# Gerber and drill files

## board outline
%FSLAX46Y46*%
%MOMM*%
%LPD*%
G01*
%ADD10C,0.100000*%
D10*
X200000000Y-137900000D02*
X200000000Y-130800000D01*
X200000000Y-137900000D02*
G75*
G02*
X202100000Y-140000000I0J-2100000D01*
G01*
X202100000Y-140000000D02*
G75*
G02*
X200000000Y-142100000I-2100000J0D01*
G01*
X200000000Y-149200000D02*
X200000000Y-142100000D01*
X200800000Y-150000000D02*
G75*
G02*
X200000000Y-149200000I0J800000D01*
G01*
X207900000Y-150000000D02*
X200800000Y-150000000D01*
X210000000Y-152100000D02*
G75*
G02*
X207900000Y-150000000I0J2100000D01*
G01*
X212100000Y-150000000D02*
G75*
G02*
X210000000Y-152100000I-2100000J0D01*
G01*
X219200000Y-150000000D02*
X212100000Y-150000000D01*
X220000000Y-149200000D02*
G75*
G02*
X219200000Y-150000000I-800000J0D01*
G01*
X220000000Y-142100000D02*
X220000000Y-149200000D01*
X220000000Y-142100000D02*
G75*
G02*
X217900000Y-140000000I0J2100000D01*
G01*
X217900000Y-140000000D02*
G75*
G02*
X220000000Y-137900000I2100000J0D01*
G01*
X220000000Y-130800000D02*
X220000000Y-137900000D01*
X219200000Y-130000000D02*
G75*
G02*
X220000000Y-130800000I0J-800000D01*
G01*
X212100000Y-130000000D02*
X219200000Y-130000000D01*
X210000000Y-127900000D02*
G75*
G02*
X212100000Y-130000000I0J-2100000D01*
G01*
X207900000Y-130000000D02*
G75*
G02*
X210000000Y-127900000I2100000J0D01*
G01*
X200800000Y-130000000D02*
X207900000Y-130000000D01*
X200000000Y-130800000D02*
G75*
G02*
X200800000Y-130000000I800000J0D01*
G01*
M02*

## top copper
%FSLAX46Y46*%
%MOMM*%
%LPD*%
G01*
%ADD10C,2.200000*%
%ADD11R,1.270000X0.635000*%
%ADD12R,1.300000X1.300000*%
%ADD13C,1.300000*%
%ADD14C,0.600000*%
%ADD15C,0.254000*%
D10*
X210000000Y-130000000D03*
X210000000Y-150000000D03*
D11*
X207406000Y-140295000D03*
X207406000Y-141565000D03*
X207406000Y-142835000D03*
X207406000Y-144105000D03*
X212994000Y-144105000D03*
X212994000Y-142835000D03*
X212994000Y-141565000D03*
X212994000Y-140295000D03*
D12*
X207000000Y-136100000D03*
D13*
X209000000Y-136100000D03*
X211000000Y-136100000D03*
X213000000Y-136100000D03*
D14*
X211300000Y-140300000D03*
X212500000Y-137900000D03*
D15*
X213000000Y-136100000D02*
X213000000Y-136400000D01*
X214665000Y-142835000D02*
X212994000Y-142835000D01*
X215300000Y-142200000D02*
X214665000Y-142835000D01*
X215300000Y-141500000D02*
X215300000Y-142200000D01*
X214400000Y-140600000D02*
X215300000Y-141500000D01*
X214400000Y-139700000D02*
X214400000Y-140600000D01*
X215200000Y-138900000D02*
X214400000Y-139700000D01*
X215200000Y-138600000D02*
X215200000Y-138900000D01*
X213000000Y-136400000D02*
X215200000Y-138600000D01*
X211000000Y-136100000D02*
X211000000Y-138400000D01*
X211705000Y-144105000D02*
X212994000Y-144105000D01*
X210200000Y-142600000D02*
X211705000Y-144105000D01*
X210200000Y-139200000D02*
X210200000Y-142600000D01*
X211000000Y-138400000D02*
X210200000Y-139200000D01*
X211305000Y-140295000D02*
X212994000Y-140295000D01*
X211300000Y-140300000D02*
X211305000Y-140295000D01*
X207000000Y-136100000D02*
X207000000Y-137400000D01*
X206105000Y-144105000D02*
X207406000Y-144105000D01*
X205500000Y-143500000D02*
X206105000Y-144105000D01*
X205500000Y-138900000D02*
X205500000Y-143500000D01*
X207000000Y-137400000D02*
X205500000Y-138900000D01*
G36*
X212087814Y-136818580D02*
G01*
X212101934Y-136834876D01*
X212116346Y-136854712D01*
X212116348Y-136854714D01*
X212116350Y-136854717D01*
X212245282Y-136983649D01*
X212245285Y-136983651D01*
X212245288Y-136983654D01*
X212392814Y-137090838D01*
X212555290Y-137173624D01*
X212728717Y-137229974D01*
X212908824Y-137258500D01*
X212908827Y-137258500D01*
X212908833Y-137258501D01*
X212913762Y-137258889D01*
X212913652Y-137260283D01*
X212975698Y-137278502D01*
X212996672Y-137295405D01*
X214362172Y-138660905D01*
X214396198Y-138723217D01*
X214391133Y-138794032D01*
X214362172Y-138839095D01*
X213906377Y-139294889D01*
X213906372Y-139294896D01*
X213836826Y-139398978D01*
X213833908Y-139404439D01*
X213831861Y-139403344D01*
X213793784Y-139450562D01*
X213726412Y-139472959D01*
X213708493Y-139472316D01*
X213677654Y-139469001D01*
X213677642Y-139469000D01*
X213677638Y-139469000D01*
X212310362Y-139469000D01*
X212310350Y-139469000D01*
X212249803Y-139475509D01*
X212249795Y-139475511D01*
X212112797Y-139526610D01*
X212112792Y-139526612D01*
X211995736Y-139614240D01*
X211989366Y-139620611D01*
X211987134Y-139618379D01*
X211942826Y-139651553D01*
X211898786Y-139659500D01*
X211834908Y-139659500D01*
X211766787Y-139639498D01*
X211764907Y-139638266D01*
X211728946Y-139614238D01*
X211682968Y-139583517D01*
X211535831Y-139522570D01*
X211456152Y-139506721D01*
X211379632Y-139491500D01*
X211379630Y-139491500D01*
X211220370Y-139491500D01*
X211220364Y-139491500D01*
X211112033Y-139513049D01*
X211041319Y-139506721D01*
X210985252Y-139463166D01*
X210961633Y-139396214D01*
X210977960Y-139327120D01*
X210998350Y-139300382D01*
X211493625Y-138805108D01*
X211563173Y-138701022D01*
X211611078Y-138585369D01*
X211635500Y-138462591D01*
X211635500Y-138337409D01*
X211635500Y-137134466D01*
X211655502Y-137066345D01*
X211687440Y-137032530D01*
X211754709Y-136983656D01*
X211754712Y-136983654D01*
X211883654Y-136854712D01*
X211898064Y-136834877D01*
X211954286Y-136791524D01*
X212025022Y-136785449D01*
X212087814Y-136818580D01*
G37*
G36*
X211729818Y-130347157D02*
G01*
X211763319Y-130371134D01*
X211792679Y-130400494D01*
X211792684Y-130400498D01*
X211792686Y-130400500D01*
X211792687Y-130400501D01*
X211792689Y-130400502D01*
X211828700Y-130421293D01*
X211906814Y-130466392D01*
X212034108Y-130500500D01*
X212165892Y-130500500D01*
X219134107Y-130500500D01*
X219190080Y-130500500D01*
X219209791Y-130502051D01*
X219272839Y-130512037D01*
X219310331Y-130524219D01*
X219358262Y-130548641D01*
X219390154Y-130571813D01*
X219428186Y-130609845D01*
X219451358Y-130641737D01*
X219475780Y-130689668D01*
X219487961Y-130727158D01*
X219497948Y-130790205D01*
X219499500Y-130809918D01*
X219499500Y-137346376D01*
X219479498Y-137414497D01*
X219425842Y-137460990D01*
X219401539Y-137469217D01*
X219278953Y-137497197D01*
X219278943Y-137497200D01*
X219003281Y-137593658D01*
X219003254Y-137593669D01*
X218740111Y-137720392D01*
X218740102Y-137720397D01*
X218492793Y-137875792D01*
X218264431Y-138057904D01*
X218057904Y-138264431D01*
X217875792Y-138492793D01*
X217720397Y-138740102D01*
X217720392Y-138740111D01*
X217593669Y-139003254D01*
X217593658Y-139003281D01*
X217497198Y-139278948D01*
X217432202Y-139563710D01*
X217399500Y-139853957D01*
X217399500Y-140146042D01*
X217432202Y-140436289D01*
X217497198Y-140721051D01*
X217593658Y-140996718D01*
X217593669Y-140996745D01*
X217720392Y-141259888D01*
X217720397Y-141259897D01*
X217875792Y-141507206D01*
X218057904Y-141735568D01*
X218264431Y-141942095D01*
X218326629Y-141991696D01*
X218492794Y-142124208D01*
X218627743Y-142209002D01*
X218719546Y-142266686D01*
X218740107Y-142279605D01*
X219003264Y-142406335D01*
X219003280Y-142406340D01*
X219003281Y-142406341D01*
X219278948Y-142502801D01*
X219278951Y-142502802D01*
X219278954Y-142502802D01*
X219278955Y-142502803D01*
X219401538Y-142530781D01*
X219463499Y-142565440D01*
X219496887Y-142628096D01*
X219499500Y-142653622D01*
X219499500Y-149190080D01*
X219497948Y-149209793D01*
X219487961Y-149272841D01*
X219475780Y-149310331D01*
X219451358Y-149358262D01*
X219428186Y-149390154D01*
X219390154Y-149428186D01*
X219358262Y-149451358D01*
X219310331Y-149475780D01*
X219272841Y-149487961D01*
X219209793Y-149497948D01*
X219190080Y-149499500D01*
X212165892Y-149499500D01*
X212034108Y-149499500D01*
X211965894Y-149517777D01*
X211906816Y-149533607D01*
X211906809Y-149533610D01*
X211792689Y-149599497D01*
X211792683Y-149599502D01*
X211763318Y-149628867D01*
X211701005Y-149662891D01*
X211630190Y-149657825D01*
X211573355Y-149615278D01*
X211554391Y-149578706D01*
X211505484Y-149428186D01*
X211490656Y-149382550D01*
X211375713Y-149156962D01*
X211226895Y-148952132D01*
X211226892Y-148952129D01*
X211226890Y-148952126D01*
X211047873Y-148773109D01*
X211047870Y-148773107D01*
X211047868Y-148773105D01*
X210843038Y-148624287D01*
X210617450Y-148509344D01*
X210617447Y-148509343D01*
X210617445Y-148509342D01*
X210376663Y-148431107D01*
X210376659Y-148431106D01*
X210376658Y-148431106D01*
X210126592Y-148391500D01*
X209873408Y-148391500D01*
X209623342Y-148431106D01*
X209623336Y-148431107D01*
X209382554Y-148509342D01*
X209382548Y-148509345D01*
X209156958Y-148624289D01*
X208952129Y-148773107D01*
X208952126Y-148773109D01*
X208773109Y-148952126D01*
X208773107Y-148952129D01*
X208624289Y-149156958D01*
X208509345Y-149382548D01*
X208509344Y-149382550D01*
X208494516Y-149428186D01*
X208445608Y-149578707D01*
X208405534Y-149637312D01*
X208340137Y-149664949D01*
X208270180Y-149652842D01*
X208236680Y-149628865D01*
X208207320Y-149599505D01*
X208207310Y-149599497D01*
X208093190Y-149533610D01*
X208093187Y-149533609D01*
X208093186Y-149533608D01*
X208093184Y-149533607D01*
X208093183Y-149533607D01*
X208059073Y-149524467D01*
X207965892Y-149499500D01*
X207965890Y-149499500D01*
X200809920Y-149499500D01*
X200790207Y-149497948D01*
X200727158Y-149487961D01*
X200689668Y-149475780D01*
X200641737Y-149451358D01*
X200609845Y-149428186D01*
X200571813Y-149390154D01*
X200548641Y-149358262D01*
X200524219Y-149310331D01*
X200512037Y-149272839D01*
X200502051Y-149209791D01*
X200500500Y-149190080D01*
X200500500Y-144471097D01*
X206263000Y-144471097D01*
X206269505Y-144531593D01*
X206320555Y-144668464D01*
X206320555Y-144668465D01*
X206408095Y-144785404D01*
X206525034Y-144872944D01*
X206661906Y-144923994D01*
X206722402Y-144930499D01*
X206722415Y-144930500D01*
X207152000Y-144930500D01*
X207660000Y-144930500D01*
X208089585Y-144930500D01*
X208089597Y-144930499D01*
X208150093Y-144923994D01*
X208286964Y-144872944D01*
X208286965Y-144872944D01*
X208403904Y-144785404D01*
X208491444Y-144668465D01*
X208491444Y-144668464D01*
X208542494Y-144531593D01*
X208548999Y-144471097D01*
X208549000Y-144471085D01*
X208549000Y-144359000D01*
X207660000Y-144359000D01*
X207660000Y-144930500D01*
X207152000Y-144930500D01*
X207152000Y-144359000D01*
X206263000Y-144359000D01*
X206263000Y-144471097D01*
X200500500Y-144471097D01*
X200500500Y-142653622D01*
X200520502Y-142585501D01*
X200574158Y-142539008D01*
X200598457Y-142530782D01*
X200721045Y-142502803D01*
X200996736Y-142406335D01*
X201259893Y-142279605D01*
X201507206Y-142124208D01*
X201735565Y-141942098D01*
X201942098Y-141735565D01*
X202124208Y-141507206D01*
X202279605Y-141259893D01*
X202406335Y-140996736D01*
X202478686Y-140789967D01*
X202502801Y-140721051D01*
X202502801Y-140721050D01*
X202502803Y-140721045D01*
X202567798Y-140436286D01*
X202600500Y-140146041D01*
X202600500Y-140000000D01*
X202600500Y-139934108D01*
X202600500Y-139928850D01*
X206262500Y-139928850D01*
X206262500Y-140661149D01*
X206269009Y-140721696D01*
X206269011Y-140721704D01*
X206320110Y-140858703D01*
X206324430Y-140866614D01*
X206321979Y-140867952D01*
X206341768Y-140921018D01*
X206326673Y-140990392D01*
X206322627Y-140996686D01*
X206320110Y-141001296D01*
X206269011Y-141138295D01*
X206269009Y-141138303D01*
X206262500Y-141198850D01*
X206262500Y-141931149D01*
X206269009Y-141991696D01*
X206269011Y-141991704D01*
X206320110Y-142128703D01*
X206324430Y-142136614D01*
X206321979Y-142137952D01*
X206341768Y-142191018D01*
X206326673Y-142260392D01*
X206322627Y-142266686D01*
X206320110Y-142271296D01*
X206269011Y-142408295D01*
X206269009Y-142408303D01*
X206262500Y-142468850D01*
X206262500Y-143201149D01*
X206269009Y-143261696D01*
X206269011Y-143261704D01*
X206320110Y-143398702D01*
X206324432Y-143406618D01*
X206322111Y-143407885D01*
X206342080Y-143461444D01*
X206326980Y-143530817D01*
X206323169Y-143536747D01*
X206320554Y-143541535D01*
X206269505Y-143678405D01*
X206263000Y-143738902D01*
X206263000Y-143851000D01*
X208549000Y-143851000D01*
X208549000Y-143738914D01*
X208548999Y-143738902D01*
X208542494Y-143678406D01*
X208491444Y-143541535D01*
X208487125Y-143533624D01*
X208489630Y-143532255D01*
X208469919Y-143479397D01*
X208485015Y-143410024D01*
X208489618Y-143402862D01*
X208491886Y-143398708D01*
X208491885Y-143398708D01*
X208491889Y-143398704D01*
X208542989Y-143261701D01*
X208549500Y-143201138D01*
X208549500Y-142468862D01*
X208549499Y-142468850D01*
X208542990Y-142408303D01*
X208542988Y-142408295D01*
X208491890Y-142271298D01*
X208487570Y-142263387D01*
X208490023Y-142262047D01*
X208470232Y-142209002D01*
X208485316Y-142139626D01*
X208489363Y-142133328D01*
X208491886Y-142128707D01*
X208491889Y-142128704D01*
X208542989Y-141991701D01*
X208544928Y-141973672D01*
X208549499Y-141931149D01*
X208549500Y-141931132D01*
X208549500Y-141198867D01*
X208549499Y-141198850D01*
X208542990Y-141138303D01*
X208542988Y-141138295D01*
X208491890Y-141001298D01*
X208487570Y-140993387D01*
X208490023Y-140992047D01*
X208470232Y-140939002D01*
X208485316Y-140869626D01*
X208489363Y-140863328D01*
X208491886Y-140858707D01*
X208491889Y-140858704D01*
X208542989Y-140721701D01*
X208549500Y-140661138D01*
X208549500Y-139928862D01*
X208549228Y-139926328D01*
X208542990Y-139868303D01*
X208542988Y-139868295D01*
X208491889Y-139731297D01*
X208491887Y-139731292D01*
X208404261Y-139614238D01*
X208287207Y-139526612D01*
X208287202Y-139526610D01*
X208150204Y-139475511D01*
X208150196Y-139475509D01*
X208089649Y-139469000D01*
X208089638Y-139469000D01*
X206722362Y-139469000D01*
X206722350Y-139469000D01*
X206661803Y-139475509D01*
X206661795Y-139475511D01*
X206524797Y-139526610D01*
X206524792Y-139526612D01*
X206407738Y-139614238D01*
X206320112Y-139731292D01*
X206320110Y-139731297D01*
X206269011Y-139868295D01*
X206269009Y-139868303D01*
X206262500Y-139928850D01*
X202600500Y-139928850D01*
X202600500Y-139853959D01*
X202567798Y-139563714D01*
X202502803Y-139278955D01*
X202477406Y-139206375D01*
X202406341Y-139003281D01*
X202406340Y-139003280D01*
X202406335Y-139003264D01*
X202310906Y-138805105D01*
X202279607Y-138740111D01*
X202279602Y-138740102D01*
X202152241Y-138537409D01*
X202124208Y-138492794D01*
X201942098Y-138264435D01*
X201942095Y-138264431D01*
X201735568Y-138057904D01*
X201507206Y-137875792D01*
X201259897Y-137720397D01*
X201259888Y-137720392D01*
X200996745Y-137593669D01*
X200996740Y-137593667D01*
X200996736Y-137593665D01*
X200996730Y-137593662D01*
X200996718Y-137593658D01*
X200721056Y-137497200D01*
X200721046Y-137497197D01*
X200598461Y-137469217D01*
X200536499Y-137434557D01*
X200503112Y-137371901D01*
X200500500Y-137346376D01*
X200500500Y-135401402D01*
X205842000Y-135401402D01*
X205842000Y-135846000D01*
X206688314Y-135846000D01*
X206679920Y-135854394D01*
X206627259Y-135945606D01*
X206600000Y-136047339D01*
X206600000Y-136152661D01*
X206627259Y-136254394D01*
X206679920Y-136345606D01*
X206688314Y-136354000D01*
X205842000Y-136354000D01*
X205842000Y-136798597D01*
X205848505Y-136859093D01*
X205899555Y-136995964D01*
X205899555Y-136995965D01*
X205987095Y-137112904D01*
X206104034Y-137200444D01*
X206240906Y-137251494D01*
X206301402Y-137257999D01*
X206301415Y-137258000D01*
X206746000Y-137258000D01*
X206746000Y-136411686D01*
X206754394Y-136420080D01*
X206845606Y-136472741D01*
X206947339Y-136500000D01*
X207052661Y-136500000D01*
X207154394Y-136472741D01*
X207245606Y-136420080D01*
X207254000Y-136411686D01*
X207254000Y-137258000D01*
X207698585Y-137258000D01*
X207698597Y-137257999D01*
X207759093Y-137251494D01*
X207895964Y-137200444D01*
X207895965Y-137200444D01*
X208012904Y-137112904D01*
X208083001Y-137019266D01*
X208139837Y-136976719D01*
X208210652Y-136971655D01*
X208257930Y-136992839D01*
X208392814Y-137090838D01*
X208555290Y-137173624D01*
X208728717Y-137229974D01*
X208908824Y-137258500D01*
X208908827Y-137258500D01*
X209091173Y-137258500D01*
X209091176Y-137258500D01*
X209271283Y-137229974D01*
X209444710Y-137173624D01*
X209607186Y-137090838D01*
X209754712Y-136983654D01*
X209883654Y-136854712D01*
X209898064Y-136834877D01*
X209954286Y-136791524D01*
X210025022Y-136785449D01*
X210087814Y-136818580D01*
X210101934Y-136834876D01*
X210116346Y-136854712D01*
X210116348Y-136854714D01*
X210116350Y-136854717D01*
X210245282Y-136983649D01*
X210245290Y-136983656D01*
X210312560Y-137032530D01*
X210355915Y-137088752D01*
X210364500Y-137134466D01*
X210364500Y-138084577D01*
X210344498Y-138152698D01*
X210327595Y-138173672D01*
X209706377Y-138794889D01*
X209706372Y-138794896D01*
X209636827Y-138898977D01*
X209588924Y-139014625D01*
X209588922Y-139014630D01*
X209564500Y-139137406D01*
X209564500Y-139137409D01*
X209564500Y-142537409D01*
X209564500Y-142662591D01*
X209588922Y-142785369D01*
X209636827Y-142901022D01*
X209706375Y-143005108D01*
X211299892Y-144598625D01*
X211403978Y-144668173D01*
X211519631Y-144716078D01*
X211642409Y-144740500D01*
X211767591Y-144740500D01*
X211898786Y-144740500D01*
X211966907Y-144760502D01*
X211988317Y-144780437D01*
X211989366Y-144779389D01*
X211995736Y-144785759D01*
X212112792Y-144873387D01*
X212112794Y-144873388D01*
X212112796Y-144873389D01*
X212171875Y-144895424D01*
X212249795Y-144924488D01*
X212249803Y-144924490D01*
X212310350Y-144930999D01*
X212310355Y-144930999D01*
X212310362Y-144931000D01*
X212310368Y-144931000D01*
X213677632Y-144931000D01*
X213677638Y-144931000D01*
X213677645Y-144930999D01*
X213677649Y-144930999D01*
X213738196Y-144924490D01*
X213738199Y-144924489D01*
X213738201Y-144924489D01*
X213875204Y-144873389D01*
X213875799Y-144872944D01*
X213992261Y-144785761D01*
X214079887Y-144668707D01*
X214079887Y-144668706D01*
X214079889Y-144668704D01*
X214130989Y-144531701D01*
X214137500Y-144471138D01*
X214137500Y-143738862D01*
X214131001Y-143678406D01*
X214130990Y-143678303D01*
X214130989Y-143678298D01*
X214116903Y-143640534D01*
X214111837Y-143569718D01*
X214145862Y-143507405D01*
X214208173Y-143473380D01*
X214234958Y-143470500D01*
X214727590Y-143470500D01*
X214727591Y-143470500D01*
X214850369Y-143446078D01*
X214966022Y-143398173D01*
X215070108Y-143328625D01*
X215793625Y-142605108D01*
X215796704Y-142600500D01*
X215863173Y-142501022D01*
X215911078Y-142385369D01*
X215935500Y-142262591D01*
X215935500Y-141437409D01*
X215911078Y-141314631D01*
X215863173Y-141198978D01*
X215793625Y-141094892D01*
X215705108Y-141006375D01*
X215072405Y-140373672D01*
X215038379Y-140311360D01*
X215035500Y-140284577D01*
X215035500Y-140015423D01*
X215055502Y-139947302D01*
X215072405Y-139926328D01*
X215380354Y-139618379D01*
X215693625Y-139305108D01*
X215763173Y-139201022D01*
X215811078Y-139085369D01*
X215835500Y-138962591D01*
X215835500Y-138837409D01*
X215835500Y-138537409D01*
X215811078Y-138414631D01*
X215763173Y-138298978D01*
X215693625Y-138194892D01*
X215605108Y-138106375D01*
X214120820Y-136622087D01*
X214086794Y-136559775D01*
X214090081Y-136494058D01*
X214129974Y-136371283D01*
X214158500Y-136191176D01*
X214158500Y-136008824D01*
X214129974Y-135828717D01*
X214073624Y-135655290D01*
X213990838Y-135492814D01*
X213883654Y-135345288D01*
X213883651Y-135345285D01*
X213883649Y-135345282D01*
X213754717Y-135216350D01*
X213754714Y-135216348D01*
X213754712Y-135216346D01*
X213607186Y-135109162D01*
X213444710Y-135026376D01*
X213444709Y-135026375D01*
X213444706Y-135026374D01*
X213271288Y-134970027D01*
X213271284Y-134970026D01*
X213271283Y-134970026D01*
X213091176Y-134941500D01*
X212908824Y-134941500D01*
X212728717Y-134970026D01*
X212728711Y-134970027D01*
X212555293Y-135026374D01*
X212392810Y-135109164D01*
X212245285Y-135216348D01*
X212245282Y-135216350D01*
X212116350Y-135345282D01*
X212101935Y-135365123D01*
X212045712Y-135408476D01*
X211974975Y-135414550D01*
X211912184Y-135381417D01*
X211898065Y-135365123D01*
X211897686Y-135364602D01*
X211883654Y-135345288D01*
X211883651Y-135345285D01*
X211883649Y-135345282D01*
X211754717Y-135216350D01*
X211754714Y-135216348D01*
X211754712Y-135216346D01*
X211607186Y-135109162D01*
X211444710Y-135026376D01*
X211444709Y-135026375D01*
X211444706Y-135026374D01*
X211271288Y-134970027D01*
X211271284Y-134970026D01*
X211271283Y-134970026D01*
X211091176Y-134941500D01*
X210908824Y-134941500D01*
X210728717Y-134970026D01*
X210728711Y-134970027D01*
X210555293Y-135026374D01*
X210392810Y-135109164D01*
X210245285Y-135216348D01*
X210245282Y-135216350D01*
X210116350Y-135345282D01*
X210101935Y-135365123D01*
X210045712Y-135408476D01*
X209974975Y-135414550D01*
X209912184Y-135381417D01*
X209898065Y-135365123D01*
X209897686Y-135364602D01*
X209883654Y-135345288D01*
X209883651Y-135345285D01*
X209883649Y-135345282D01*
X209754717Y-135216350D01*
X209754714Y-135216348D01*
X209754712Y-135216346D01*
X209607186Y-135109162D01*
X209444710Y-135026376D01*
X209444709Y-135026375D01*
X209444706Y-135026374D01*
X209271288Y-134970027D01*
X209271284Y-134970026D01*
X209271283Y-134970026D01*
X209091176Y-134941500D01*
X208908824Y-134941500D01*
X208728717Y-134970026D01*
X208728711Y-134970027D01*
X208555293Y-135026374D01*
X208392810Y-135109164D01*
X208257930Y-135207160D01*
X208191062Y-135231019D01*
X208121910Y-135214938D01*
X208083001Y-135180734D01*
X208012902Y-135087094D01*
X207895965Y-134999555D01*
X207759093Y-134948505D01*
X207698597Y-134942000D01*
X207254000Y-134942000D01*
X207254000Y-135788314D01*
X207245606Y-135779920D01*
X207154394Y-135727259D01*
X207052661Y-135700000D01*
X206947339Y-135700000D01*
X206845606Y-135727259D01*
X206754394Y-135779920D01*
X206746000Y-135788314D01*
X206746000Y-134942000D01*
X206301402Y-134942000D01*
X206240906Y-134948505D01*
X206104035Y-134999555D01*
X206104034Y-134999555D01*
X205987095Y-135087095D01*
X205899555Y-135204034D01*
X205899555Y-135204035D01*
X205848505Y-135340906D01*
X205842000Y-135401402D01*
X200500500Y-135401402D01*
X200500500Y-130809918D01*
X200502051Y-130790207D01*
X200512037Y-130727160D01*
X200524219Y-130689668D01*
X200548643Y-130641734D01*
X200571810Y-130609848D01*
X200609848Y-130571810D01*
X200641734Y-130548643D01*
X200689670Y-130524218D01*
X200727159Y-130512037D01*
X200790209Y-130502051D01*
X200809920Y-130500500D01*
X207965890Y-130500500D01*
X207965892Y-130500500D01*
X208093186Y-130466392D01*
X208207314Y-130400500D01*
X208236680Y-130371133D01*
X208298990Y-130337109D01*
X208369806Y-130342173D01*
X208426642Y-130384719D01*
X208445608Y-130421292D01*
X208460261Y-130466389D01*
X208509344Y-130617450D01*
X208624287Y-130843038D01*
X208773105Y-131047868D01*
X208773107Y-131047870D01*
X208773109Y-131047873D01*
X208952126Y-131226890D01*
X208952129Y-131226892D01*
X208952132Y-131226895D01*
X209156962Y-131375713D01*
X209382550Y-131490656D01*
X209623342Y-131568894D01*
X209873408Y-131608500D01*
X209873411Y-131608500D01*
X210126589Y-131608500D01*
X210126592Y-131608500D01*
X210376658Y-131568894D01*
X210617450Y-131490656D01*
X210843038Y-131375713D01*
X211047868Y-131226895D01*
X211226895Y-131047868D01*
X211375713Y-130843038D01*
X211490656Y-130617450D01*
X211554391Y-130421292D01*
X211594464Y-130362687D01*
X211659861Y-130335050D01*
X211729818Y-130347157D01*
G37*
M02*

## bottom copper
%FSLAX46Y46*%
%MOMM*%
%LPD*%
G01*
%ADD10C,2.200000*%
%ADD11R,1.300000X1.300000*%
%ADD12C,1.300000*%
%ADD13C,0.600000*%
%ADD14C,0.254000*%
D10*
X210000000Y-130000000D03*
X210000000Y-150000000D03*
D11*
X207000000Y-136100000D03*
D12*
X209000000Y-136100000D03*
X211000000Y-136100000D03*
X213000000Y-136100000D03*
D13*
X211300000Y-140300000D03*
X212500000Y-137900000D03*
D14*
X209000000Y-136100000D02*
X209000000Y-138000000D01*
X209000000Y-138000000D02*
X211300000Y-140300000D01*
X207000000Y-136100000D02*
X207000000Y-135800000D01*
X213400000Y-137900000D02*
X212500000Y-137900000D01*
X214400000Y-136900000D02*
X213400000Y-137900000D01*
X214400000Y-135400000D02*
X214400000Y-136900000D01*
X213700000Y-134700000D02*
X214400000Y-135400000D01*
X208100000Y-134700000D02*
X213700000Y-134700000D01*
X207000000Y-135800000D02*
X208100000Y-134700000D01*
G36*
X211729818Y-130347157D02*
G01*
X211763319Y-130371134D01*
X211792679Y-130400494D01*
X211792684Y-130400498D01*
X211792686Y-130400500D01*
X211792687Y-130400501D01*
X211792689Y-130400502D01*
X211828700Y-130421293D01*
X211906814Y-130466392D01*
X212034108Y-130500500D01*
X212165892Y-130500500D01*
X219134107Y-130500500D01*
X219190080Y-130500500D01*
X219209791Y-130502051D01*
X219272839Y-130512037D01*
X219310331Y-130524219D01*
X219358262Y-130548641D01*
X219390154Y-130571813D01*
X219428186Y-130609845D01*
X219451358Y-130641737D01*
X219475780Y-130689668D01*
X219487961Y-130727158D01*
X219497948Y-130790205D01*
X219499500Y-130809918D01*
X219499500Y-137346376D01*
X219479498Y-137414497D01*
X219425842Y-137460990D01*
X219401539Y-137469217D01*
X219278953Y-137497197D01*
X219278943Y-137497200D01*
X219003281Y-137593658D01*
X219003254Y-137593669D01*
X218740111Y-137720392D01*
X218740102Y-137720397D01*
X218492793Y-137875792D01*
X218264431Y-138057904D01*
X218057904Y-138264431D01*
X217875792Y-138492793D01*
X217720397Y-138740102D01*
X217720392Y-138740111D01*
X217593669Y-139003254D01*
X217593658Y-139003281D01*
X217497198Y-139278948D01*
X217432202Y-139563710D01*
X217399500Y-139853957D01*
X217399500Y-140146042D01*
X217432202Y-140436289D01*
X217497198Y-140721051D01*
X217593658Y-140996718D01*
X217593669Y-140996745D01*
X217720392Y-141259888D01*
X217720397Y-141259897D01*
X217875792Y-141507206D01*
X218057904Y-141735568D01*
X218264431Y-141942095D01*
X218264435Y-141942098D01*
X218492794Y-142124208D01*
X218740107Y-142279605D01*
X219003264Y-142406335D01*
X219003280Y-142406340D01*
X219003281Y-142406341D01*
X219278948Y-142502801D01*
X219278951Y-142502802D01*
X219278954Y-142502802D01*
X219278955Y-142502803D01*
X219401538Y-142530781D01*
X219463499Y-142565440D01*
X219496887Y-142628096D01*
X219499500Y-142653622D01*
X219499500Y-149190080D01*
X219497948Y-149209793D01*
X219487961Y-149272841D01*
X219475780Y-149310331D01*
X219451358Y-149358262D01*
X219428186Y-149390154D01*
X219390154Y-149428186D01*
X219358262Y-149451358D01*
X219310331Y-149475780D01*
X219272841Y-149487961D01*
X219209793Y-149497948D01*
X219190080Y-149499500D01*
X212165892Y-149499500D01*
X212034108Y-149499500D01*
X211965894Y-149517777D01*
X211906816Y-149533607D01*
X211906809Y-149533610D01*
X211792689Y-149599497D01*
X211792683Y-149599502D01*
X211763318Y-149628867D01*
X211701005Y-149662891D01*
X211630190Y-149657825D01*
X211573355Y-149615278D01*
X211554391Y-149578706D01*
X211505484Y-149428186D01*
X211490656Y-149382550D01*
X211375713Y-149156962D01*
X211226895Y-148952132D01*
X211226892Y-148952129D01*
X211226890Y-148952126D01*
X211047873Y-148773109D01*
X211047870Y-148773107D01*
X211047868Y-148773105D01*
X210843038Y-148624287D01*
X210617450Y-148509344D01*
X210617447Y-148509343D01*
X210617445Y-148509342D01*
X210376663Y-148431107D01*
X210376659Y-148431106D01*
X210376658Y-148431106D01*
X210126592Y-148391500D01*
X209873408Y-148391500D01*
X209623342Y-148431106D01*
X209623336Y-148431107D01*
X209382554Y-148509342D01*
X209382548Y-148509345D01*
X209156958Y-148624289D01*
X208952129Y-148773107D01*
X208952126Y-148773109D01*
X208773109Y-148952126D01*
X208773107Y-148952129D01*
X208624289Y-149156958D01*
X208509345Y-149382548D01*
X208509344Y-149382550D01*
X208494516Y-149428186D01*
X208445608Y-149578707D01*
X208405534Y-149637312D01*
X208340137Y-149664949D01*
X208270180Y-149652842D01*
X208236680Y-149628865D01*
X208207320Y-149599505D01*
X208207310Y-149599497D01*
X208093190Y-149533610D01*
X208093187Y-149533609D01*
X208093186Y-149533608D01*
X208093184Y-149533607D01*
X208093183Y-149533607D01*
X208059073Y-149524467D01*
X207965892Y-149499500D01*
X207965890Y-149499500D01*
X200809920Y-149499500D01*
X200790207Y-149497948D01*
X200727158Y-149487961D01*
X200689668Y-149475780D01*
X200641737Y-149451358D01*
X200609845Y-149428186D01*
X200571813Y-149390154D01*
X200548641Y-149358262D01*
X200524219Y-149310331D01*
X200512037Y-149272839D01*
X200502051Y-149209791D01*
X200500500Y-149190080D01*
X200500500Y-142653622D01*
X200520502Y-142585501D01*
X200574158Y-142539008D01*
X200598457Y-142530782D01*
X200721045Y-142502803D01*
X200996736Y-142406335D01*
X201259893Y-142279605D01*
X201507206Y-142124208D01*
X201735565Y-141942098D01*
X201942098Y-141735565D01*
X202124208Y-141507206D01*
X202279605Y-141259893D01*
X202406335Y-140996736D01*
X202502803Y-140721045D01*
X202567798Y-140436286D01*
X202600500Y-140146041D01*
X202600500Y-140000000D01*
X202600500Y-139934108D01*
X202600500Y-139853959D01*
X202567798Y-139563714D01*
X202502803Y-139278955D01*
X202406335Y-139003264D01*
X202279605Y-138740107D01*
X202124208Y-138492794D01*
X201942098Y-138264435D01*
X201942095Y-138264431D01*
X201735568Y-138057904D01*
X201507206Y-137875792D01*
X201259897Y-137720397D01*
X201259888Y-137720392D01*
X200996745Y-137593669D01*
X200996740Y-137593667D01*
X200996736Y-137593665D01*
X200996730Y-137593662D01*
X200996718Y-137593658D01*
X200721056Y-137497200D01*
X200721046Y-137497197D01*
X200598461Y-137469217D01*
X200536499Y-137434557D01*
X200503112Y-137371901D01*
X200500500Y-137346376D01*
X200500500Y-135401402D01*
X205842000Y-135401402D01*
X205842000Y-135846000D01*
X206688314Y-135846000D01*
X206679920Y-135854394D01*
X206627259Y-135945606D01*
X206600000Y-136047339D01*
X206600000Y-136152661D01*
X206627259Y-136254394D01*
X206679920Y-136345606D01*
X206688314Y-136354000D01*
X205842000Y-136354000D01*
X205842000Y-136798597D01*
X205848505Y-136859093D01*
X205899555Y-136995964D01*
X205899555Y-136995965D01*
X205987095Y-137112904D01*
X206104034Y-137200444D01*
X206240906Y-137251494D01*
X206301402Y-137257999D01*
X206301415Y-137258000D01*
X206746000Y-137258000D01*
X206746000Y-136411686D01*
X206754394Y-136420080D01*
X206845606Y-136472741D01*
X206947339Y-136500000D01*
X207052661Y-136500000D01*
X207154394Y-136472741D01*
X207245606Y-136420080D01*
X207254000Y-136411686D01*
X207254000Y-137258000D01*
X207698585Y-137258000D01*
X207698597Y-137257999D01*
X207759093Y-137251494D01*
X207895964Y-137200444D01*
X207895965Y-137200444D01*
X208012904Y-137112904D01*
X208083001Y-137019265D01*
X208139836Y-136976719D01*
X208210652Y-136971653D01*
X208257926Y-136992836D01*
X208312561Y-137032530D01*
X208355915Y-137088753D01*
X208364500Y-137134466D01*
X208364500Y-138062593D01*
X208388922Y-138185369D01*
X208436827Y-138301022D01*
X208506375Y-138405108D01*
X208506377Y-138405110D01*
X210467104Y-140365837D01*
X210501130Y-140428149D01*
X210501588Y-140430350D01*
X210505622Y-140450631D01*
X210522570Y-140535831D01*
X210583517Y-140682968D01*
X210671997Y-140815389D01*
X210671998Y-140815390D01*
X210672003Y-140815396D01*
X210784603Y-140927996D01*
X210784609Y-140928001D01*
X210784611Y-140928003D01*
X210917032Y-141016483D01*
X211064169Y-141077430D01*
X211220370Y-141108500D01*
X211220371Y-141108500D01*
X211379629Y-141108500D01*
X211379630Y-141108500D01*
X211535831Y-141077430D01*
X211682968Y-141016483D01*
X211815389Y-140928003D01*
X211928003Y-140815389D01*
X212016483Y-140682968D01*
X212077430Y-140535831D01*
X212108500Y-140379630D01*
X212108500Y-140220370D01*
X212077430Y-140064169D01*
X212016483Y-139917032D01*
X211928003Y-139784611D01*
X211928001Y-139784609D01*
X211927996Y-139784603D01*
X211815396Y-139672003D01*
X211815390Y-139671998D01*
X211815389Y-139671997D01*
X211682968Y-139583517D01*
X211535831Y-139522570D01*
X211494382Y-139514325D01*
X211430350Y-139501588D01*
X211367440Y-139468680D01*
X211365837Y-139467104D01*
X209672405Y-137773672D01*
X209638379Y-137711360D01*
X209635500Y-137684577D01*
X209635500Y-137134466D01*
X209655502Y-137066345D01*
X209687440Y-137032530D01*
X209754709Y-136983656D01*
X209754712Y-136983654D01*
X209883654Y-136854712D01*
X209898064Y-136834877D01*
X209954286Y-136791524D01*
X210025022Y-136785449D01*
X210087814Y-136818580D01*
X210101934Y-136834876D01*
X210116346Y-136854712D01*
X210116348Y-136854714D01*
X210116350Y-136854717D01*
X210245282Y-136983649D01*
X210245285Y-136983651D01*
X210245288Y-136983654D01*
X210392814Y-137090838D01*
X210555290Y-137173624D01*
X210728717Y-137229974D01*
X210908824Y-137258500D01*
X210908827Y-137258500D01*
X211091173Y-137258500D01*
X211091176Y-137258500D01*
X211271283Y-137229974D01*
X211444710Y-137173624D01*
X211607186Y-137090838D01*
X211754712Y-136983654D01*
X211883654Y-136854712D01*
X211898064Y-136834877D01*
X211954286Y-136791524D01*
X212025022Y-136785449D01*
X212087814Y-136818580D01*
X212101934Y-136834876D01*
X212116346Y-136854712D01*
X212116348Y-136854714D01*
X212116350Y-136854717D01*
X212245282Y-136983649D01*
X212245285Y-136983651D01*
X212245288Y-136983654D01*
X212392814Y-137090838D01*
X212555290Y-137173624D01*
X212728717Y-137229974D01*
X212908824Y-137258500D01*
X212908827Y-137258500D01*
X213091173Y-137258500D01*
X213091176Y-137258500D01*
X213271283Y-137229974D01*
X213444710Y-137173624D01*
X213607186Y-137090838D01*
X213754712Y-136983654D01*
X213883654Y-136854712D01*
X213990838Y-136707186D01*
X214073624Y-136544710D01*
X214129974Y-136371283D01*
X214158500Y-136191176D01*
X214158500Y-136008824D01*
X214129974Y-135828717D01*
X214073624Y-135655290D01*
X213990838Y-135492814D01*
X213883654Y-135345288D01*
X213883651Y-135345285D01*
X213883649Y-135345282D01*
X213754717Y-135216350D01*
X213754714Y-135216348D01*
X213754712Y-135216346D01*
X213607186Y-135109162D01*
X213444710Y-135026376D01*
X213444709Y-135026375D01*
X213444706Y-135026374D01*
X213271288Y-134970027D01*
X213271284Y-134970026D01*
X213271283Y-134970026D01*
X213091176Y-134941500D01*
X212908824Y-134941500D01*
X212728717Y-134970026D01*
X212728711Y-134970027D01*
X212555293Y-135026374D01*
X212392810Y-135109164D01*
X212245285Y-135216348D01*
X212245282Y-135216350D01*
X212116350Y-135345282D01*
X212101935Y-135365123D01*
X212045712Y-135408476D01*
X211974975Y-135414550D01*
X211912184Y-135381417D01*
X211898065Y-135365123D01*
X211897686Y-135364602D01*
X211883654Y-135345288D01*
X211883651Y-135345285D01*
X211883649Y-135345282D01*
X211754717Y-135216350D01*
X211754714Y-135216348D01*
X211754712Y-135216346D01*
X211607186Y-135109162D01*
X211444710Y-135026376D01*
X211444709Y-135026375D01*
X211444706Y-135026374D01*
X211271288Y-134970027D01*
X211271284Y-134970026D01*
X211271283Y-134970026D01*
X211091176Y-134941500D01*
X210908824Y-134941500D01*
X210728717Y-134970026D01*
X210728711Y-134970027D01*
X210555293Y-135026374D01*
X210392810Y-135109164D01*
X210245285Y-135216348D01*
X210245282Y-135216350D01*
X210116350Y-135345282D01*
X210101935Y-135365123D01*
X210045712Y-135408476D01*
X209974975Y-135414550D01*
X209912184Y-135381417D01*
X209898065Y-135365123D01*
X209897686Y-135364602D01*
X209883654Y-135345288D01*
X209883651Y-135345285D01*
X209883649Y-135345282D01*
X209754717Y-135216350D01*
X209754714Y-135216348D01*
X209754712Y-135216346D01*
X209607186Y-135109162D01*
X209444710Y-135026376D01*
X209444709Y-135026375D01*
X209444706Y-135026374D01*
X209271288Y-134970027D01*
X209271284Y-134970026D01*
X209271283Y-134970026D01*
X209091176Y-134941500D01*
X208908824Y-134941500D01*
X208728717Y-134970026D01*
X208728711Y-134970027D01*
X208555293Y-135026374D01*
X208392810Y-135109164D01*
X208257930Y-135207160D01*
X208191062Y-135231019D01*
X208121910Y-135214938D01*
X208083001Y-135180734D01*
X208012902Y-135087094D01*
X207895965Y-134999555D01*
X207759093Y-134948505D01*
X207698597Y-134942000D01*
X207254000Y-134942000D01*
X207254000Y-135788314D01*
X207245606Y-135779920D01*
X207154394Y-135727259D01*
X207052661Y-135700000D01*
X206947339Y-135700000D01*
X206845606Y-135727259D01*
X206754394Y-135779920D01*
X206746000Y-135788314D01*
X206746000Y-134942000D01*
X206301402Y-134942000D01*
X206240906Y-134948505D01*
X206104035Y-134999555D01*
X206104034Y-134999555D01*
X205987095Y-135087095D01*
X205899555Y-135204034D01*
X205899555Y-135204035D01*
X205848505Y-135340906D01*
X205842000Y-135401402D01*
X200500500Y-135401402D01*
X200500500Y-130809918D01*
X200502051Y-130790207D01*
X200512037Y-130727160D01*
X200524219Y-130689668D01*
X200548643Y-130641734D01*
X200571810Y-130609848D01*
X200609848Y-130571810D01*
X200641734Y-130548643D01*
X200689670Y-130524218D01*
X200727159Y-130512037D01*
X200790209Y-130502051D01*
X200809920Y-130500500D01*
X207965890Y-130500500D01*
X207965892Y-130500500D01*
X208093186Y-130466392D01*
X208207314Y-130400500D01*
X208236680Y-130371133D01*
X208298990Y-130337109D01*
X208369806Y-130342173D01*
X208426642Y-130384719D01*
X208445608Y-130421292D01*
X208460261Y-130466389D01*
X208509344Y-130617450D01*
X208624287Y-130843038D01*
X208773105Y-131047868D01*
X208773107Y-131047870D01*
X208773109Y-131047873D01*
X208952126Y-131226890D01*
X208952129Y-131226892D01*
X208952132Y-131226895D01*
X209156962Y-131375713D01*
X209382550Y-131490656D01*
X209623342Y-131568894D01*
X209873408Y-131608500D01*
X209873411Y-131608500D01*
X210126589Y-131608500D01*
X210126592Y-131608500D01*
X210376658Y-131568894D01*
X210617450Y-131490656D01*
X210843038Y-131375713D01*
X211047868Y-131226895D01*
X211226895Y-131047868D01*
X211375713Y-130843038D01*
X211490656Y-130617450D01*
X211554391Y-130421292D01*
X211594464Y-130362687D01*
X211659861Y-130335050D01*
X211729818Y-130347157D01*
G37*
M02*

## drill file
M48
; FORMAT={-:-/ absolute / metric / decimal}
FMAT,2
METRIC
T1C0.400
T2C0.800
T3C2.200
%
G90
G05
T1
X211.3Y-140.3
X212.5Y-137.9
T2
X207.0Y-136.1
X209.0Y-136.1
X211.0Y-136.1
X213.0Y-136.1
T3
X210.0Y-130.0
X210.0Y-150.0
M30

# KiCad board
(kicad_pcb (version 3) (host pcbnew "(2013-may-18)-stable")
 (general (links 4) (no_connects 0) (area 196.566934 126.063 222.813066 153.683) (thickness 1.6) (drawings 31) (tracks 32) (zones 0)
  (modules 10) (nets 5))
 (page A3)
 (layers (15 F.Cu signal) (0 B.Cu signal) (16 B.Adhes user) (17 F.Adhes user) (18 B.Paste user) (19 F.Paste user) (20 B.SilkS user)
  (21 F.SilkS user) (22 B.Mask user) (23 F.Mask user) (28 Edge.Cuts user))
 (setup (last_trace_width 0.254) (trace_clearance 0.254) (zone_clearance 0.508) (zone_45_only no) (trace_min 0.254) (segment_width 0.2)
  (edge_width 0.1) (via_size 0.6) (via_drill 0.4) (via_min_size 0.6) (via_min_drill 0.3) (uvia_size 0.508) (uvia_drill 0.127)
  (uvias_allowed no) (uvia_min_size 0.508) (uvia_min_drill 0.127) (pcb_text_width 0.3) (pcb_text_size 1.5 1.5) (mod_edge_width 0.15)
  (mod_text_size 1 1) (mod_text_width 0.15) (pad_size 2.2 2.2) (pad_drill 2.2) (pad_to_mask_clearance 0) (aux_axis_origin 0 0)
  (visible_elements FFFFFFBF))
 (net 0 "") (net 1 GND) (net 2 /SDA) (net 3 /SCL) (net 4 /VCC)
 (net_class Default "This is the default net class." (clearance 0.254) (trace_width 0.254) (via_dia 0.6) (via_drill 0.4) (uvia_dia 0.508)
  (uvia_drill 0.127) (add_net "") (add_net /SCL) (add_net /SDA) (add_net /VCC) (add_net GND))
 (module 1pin (layer F.Cu) (at 210 130)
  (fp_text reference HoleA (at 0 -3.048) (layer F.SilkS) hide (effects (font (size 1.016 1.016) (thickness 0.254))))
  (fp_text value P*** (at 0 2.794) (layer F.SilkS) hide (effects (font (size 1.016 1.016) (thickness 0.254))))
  (pad 1 thru_hole circle (at 0 0) (size 2.2 2.2) (drill 2.2) (layers *.Cu *.Mask F.SilkS)))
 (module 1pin (layer F.Cu) (at 210 150)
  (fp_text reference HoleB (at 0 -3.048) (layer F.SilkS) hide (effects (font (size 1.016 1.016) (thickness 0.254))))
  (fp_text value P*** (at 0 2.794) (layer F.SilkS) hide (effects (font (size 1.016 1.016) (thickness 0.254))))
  (pad 1 thru_hole circle (at 0 0) (size 2.2 2.2) (drill 2.2) (layers *.Cu *.Mask F.SilkS)))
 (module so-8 (layer F.Cu) (at 210.2 142.2 270)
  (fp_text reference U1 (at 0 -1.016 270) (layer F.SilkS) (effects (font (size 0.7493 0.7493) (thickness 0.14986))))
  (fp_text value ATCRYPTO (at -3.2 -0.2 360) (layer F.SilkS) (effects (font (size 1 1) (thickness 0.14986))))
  (pad 1 smd rect (at -1.905 2.794 270) (size 0.635 1.27) (layers F.Cu F.Paste F.Mask))
  (pad 2 smd rect (at -0.635 2.794 270) (size 0.635 1.27) (layers F.Cu F.Paste F.Mask))
  (pad 3 smd rect (at 0.635 2.794 270) (size 0.635 1.27) (layers F.Cu F.Paste F.Mask))
  (pad 4 smd rect (at 1.905 2.794 270) (size 0.635 1.27) (layers F.Cu F.Paste F.Mask) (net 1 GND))
  (pad 5 smd rect (at 1.905 -2.794 270) (size 0.635 1.27) (layers F.Cu F.Paste F.Mask) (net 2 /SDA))
  (pad 6 smd rect (at 0.635 -2.794 270) (size 0.635 1.27) (layers F.Cu F.Paste F.Mask) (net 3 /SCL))
  (pad 7 smd rect (at -0.635 -2.794 270) (size 0.635 1.27) (layers F.Cu F.Paste F.Mask))
  (pad 8 smd rect (at -1.905 -2.794 270) (size 0.635 1.27) (layers F.Cu F.Paste F.Mask) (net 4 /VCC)))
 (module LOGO (layer B.Cu) (at 215.9 146.7)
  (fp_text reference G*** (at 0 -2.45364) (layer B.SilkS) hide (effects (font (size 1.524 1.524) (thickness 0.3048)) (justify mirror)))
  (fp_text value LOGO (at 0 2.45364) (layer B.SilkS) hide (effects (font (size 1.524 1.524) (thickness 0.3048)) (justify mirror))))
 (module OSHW (layer B.Cu) (at 216.3 133.2)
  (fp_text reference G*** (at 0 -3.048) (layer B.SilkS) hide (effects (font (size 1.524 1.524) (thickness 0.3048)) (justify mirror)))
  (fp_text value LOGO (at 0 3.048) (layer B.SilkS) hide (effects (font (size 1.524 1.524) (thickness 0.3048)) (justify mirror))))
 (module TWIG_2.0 (layer F.Cu) (at 210 136.1)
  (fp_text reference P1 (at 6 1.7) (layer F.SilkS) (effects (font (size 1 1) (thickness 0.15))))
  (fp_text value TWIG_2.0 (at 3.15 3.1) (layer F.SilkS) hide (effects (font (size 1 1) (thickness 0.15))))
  (pad 1 thru_hole rect (at -3 0) (size 1.3 1.3) (drill 0.8) (layers *.Cu *.Mask F.SilkS) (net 1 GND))
  (pad 2 thru_hole circle (at -1 0) (size 1.3 1.3) (drill 0.8) (layers *.Cu *.Mask F.SilkS) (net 4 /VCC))
  (pad 3 thru_hole circle (at 1 0) (size 1.3 1.3) (drill 0.8) (layers *.Cu *.Mask F.SilkS) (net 2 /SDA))
  (pad 4 thru_hole circle (at 3 0) (size 1.3 1.3) (drill 0.8) (layers *.Cu *.Mask F.SilkS) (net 3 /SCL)))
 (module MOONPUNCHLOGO (layer B.Cu) (at 211.4 141.4)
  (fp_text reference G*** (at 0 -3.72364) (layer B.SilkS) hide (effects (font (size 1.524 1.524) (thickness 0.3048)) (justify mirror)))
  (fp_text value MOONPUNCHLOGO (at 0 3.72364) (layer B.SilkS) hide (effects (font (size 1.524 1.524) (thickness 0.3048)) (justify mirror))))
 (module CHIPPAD (layer F.Cu) (at 202.9 147.5)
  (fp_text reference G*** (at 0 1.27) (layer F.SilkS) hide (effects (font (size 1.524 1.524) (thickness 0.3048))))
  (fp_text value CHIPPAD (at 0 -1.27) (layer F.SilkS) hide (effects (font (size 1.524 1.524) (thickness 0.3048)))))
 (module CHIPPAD (layer F.Cu) (at 209.1 147.5)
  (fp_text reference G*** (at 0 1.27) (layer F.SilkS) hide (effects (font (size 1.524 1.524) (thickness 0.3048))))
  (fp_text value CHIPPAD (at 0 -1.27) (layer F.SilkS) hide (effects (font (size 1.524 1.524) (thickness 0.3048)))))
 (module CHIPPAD (layer F.Cu) (at 215 147.5)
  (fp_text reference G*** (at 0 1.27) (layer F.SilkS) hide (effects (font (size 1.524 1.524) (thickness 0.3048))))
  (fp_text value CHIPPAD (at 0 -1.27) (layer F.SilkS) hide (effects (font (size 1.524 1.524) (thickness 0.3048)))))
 (gr_line (start 200 137.9) (end 200 130.8) (angle 90) (layer Edge.Cuts) (width 0.1))
 (gr_arc (start 200 140) (end 200 137.9) (angle 90) (layer Edge.Cuts) (width 0.1))
 (gr_arc (start 200 140) (end 202.1 140) (angle 90) (layer Edge.Cuts) (width 0.1))
 (gr_line (start 200 149.2) (end 200 142.1) (angle 90) (layer Edge.Cuts) (width 0.1))
 (gr_arc (start 200.8 149.2) (end 200.8 150) (angle 90) (layer Edge.Cuts) (width 0.1))
 (gr_line (start 207.9 150) (end 200.8 150) (angle 90) (layer Edge.Cuts) (width 0.1))
 (gr_arc (start 210 150) (end 210 152.1) (angle 90) (layer Edge.Cuts) (width 0.1))
 (gr_arc (start 210 150) (end 212.1 150) (angle 90) (layer Edge.Cuts) (width 0.1))
 (gr_line (start 219.2 150) (end 212.1 150) (angle 90) (layer Edge.Cuts) (width 0.1))
 (gr_arc (start 219.2 149.2) (end 220 149.2) (angle 90) (layer Edge.Cuts) (width 0.1))
 (gr_line (start 220 142.1) (end 220 149.2) (angle 90) (layer Edge.Cuts) (width 0.1))
 (gr_arc (start 220 140) (end 220 142.1) (angle 90) (layer Edge.Cuts) (width 0.1))
 (gr_arc (start 220 140) (end 217.9 140) (angle 90) (layer Edge.Cuts) (width 0.1))
 (gr_line (start 220 130.8) (end 220 137.9) (angle 90) (layer Edge.Cuts) (width 0.1))
 (gr_arc (start 219.2 130.8) (end 219.2 130) (angle 90) (layer Edge.Cuts) (width 0.1))
 (gr_line (start 212.1 130) (end 219.2 130) (angle 90) (layer Edge.Cuts) (width 0.1))
 (gr_arc (start 210 130) (end 210 127.9) (angle 90) (layer Edge.Cuts) (width 0.1))
 (gr_arc (start 210 130) (end 207.9 130) (angle 90) (layer Edge.Cuts) (width 0.1))
 (gr_line (start 200.8 130) (end 207.9 130) (angle 90) (layer Edge.Cuts) (width 0.1))
 (gr_arc (start 200.8 130.8) (end 200 130.8) (angle 90) (layer Edge.Cuts) (width 0.1))
 (segment (start 213 136.1) (end 213 136.4) (width 0.254) (layer F.Cu) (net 3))
 (segment (start 214.665 142.835) (end 212.994 142.835) (width 0.254) (layer F.Cu) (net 3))
 (segment (start 215.3 142.2) (end 214.665 142.835) (width 0.254) (layer F.Cu) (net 3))
 (segment (start 215.3 141.5) (end 215.3 142.2) (width 0.254) (layer F.Cu) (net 3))
 (segment (start 214.4 140.6) (end 215.3 141.5) (width 0.254) (layer F.Cu) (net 3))
 (segment (start 214.4 139.7) (end 214.4 140.6) (width 0.254) (layer F.Cu) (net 3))
 (segment (start 215.2 138.9) (end 214.4 139.7) (width 0.254) (layer F.Cu) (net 3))
 (segment (start 215.2 138.6) (end 215.2 138.9) (width 0.254) (layer F.Cu) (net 3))
 (segment (start 213 136.4) (end 215.2 138.6) (width 0.254) (layer F.Cu) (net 3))
 (segment (start 211 136.1) (end 211 138.4) (width 0.254) (layer F.Cu) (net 2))
 (segment (start 211.705 144.105) (end 212.994 144.105) (width 0.254) (layer F.Cu) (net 2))
 (segment (start 210.2 142.6) (end 211.705 144.105) (width 0.254) (layer F.Cu) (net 2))
 (segment (start 210.2 139.2) (end 210.2 142.6) (width 0.254) (layer F.Cu) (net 2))
 (segment (start 211 138.4) (end 210.2 139.2) (width 0.254) (layer F.Cu) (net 2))
 (segment (start 209 136.1) (end 209 138) (width 0.254) (layer B.Cu) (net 4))
 (segment (start 211.305 140.295) (end 212.994 140.295) (width 0.254) (layer F.Cu) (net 4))
 (segment (start 211.3 140.3) (end 211.305 140.295) (width 0.254) (layer F.Cu) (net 4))
 (via (at 211.3 140.3) (size 0.6) (layers F.Cu B.Cu) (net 4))
 (segment (start 209 138) (end 211.3 140.3) (width 0.254) (layer B.Cu) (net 4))
 (segment (start 207 136.1) (end 207 135.8) (width 0.254) (layer B.Cu) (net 1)) (via (at 212.5 137.9) (size 0.6) (layers F.Cu B.Cu) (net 1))
 (segment (start 213.4 137.9) (end 212.5 137.9) (width 0.254) (layer B.Cu) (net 1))
 (segment (start 214.4 136.9) (end 213.4 137.9) (width 0.254) (layer B.Cu) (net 1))
 (segment (start 214.4 135.4) (end 214.4 136.9) (width 0.254) (layer B.Cu) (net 1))
 (segment (start 213.7 134.7) (end 214.4 135.4) (width 0.254) (layer B.Cu) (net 1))
 (segment (start 208.1 134.7) (end 213.7 134.7) (width 0.254) (layer B.Cu) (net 1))
 (segment (start 207 135.8) (end 208.1 134.7) (width 0.254) (layer B.Cu) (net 1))
 (segment (start 207 136.1) (end 207 137.4) (width 0.254) (layer F.Cu) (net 1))
 (segment (start 206.105 144.105) (end 207.406 144.105) (width 0.254) (layer F.Cu) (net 1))
 (segment (start 205.5 143.5) (end 206.105 144.105) (width 0.254) (layer F.Cu) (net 1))
 (segment (start 205.5 138.9) (end 205.5 143.5) (width 0.254) (layer F.Cu) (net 1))
 (segment (start 207 137.4) (end 205.5 138.9) (width 0.254) (layer F.Cu) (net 1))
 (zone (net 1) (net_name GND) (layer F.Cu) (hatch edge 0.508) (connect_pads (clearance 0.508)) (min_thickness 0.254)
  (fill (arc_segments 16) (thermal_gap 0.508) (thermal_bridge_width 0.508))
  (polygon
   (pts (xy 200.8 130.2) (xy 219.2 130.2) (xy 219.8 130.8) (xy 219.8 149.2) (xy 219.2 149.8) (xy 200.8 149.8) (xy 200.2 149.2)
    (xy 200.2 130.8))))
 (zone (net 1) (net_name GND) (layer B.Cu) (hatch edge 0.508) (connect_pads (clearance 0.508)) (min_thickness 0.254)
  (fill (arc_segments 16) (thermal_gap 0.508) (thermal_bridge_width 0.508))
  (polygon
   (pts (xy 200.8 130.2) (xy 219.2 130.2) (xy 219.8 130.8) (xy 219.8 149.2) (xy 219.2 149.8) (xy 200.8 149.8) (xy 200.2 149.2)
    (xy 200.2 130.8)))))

